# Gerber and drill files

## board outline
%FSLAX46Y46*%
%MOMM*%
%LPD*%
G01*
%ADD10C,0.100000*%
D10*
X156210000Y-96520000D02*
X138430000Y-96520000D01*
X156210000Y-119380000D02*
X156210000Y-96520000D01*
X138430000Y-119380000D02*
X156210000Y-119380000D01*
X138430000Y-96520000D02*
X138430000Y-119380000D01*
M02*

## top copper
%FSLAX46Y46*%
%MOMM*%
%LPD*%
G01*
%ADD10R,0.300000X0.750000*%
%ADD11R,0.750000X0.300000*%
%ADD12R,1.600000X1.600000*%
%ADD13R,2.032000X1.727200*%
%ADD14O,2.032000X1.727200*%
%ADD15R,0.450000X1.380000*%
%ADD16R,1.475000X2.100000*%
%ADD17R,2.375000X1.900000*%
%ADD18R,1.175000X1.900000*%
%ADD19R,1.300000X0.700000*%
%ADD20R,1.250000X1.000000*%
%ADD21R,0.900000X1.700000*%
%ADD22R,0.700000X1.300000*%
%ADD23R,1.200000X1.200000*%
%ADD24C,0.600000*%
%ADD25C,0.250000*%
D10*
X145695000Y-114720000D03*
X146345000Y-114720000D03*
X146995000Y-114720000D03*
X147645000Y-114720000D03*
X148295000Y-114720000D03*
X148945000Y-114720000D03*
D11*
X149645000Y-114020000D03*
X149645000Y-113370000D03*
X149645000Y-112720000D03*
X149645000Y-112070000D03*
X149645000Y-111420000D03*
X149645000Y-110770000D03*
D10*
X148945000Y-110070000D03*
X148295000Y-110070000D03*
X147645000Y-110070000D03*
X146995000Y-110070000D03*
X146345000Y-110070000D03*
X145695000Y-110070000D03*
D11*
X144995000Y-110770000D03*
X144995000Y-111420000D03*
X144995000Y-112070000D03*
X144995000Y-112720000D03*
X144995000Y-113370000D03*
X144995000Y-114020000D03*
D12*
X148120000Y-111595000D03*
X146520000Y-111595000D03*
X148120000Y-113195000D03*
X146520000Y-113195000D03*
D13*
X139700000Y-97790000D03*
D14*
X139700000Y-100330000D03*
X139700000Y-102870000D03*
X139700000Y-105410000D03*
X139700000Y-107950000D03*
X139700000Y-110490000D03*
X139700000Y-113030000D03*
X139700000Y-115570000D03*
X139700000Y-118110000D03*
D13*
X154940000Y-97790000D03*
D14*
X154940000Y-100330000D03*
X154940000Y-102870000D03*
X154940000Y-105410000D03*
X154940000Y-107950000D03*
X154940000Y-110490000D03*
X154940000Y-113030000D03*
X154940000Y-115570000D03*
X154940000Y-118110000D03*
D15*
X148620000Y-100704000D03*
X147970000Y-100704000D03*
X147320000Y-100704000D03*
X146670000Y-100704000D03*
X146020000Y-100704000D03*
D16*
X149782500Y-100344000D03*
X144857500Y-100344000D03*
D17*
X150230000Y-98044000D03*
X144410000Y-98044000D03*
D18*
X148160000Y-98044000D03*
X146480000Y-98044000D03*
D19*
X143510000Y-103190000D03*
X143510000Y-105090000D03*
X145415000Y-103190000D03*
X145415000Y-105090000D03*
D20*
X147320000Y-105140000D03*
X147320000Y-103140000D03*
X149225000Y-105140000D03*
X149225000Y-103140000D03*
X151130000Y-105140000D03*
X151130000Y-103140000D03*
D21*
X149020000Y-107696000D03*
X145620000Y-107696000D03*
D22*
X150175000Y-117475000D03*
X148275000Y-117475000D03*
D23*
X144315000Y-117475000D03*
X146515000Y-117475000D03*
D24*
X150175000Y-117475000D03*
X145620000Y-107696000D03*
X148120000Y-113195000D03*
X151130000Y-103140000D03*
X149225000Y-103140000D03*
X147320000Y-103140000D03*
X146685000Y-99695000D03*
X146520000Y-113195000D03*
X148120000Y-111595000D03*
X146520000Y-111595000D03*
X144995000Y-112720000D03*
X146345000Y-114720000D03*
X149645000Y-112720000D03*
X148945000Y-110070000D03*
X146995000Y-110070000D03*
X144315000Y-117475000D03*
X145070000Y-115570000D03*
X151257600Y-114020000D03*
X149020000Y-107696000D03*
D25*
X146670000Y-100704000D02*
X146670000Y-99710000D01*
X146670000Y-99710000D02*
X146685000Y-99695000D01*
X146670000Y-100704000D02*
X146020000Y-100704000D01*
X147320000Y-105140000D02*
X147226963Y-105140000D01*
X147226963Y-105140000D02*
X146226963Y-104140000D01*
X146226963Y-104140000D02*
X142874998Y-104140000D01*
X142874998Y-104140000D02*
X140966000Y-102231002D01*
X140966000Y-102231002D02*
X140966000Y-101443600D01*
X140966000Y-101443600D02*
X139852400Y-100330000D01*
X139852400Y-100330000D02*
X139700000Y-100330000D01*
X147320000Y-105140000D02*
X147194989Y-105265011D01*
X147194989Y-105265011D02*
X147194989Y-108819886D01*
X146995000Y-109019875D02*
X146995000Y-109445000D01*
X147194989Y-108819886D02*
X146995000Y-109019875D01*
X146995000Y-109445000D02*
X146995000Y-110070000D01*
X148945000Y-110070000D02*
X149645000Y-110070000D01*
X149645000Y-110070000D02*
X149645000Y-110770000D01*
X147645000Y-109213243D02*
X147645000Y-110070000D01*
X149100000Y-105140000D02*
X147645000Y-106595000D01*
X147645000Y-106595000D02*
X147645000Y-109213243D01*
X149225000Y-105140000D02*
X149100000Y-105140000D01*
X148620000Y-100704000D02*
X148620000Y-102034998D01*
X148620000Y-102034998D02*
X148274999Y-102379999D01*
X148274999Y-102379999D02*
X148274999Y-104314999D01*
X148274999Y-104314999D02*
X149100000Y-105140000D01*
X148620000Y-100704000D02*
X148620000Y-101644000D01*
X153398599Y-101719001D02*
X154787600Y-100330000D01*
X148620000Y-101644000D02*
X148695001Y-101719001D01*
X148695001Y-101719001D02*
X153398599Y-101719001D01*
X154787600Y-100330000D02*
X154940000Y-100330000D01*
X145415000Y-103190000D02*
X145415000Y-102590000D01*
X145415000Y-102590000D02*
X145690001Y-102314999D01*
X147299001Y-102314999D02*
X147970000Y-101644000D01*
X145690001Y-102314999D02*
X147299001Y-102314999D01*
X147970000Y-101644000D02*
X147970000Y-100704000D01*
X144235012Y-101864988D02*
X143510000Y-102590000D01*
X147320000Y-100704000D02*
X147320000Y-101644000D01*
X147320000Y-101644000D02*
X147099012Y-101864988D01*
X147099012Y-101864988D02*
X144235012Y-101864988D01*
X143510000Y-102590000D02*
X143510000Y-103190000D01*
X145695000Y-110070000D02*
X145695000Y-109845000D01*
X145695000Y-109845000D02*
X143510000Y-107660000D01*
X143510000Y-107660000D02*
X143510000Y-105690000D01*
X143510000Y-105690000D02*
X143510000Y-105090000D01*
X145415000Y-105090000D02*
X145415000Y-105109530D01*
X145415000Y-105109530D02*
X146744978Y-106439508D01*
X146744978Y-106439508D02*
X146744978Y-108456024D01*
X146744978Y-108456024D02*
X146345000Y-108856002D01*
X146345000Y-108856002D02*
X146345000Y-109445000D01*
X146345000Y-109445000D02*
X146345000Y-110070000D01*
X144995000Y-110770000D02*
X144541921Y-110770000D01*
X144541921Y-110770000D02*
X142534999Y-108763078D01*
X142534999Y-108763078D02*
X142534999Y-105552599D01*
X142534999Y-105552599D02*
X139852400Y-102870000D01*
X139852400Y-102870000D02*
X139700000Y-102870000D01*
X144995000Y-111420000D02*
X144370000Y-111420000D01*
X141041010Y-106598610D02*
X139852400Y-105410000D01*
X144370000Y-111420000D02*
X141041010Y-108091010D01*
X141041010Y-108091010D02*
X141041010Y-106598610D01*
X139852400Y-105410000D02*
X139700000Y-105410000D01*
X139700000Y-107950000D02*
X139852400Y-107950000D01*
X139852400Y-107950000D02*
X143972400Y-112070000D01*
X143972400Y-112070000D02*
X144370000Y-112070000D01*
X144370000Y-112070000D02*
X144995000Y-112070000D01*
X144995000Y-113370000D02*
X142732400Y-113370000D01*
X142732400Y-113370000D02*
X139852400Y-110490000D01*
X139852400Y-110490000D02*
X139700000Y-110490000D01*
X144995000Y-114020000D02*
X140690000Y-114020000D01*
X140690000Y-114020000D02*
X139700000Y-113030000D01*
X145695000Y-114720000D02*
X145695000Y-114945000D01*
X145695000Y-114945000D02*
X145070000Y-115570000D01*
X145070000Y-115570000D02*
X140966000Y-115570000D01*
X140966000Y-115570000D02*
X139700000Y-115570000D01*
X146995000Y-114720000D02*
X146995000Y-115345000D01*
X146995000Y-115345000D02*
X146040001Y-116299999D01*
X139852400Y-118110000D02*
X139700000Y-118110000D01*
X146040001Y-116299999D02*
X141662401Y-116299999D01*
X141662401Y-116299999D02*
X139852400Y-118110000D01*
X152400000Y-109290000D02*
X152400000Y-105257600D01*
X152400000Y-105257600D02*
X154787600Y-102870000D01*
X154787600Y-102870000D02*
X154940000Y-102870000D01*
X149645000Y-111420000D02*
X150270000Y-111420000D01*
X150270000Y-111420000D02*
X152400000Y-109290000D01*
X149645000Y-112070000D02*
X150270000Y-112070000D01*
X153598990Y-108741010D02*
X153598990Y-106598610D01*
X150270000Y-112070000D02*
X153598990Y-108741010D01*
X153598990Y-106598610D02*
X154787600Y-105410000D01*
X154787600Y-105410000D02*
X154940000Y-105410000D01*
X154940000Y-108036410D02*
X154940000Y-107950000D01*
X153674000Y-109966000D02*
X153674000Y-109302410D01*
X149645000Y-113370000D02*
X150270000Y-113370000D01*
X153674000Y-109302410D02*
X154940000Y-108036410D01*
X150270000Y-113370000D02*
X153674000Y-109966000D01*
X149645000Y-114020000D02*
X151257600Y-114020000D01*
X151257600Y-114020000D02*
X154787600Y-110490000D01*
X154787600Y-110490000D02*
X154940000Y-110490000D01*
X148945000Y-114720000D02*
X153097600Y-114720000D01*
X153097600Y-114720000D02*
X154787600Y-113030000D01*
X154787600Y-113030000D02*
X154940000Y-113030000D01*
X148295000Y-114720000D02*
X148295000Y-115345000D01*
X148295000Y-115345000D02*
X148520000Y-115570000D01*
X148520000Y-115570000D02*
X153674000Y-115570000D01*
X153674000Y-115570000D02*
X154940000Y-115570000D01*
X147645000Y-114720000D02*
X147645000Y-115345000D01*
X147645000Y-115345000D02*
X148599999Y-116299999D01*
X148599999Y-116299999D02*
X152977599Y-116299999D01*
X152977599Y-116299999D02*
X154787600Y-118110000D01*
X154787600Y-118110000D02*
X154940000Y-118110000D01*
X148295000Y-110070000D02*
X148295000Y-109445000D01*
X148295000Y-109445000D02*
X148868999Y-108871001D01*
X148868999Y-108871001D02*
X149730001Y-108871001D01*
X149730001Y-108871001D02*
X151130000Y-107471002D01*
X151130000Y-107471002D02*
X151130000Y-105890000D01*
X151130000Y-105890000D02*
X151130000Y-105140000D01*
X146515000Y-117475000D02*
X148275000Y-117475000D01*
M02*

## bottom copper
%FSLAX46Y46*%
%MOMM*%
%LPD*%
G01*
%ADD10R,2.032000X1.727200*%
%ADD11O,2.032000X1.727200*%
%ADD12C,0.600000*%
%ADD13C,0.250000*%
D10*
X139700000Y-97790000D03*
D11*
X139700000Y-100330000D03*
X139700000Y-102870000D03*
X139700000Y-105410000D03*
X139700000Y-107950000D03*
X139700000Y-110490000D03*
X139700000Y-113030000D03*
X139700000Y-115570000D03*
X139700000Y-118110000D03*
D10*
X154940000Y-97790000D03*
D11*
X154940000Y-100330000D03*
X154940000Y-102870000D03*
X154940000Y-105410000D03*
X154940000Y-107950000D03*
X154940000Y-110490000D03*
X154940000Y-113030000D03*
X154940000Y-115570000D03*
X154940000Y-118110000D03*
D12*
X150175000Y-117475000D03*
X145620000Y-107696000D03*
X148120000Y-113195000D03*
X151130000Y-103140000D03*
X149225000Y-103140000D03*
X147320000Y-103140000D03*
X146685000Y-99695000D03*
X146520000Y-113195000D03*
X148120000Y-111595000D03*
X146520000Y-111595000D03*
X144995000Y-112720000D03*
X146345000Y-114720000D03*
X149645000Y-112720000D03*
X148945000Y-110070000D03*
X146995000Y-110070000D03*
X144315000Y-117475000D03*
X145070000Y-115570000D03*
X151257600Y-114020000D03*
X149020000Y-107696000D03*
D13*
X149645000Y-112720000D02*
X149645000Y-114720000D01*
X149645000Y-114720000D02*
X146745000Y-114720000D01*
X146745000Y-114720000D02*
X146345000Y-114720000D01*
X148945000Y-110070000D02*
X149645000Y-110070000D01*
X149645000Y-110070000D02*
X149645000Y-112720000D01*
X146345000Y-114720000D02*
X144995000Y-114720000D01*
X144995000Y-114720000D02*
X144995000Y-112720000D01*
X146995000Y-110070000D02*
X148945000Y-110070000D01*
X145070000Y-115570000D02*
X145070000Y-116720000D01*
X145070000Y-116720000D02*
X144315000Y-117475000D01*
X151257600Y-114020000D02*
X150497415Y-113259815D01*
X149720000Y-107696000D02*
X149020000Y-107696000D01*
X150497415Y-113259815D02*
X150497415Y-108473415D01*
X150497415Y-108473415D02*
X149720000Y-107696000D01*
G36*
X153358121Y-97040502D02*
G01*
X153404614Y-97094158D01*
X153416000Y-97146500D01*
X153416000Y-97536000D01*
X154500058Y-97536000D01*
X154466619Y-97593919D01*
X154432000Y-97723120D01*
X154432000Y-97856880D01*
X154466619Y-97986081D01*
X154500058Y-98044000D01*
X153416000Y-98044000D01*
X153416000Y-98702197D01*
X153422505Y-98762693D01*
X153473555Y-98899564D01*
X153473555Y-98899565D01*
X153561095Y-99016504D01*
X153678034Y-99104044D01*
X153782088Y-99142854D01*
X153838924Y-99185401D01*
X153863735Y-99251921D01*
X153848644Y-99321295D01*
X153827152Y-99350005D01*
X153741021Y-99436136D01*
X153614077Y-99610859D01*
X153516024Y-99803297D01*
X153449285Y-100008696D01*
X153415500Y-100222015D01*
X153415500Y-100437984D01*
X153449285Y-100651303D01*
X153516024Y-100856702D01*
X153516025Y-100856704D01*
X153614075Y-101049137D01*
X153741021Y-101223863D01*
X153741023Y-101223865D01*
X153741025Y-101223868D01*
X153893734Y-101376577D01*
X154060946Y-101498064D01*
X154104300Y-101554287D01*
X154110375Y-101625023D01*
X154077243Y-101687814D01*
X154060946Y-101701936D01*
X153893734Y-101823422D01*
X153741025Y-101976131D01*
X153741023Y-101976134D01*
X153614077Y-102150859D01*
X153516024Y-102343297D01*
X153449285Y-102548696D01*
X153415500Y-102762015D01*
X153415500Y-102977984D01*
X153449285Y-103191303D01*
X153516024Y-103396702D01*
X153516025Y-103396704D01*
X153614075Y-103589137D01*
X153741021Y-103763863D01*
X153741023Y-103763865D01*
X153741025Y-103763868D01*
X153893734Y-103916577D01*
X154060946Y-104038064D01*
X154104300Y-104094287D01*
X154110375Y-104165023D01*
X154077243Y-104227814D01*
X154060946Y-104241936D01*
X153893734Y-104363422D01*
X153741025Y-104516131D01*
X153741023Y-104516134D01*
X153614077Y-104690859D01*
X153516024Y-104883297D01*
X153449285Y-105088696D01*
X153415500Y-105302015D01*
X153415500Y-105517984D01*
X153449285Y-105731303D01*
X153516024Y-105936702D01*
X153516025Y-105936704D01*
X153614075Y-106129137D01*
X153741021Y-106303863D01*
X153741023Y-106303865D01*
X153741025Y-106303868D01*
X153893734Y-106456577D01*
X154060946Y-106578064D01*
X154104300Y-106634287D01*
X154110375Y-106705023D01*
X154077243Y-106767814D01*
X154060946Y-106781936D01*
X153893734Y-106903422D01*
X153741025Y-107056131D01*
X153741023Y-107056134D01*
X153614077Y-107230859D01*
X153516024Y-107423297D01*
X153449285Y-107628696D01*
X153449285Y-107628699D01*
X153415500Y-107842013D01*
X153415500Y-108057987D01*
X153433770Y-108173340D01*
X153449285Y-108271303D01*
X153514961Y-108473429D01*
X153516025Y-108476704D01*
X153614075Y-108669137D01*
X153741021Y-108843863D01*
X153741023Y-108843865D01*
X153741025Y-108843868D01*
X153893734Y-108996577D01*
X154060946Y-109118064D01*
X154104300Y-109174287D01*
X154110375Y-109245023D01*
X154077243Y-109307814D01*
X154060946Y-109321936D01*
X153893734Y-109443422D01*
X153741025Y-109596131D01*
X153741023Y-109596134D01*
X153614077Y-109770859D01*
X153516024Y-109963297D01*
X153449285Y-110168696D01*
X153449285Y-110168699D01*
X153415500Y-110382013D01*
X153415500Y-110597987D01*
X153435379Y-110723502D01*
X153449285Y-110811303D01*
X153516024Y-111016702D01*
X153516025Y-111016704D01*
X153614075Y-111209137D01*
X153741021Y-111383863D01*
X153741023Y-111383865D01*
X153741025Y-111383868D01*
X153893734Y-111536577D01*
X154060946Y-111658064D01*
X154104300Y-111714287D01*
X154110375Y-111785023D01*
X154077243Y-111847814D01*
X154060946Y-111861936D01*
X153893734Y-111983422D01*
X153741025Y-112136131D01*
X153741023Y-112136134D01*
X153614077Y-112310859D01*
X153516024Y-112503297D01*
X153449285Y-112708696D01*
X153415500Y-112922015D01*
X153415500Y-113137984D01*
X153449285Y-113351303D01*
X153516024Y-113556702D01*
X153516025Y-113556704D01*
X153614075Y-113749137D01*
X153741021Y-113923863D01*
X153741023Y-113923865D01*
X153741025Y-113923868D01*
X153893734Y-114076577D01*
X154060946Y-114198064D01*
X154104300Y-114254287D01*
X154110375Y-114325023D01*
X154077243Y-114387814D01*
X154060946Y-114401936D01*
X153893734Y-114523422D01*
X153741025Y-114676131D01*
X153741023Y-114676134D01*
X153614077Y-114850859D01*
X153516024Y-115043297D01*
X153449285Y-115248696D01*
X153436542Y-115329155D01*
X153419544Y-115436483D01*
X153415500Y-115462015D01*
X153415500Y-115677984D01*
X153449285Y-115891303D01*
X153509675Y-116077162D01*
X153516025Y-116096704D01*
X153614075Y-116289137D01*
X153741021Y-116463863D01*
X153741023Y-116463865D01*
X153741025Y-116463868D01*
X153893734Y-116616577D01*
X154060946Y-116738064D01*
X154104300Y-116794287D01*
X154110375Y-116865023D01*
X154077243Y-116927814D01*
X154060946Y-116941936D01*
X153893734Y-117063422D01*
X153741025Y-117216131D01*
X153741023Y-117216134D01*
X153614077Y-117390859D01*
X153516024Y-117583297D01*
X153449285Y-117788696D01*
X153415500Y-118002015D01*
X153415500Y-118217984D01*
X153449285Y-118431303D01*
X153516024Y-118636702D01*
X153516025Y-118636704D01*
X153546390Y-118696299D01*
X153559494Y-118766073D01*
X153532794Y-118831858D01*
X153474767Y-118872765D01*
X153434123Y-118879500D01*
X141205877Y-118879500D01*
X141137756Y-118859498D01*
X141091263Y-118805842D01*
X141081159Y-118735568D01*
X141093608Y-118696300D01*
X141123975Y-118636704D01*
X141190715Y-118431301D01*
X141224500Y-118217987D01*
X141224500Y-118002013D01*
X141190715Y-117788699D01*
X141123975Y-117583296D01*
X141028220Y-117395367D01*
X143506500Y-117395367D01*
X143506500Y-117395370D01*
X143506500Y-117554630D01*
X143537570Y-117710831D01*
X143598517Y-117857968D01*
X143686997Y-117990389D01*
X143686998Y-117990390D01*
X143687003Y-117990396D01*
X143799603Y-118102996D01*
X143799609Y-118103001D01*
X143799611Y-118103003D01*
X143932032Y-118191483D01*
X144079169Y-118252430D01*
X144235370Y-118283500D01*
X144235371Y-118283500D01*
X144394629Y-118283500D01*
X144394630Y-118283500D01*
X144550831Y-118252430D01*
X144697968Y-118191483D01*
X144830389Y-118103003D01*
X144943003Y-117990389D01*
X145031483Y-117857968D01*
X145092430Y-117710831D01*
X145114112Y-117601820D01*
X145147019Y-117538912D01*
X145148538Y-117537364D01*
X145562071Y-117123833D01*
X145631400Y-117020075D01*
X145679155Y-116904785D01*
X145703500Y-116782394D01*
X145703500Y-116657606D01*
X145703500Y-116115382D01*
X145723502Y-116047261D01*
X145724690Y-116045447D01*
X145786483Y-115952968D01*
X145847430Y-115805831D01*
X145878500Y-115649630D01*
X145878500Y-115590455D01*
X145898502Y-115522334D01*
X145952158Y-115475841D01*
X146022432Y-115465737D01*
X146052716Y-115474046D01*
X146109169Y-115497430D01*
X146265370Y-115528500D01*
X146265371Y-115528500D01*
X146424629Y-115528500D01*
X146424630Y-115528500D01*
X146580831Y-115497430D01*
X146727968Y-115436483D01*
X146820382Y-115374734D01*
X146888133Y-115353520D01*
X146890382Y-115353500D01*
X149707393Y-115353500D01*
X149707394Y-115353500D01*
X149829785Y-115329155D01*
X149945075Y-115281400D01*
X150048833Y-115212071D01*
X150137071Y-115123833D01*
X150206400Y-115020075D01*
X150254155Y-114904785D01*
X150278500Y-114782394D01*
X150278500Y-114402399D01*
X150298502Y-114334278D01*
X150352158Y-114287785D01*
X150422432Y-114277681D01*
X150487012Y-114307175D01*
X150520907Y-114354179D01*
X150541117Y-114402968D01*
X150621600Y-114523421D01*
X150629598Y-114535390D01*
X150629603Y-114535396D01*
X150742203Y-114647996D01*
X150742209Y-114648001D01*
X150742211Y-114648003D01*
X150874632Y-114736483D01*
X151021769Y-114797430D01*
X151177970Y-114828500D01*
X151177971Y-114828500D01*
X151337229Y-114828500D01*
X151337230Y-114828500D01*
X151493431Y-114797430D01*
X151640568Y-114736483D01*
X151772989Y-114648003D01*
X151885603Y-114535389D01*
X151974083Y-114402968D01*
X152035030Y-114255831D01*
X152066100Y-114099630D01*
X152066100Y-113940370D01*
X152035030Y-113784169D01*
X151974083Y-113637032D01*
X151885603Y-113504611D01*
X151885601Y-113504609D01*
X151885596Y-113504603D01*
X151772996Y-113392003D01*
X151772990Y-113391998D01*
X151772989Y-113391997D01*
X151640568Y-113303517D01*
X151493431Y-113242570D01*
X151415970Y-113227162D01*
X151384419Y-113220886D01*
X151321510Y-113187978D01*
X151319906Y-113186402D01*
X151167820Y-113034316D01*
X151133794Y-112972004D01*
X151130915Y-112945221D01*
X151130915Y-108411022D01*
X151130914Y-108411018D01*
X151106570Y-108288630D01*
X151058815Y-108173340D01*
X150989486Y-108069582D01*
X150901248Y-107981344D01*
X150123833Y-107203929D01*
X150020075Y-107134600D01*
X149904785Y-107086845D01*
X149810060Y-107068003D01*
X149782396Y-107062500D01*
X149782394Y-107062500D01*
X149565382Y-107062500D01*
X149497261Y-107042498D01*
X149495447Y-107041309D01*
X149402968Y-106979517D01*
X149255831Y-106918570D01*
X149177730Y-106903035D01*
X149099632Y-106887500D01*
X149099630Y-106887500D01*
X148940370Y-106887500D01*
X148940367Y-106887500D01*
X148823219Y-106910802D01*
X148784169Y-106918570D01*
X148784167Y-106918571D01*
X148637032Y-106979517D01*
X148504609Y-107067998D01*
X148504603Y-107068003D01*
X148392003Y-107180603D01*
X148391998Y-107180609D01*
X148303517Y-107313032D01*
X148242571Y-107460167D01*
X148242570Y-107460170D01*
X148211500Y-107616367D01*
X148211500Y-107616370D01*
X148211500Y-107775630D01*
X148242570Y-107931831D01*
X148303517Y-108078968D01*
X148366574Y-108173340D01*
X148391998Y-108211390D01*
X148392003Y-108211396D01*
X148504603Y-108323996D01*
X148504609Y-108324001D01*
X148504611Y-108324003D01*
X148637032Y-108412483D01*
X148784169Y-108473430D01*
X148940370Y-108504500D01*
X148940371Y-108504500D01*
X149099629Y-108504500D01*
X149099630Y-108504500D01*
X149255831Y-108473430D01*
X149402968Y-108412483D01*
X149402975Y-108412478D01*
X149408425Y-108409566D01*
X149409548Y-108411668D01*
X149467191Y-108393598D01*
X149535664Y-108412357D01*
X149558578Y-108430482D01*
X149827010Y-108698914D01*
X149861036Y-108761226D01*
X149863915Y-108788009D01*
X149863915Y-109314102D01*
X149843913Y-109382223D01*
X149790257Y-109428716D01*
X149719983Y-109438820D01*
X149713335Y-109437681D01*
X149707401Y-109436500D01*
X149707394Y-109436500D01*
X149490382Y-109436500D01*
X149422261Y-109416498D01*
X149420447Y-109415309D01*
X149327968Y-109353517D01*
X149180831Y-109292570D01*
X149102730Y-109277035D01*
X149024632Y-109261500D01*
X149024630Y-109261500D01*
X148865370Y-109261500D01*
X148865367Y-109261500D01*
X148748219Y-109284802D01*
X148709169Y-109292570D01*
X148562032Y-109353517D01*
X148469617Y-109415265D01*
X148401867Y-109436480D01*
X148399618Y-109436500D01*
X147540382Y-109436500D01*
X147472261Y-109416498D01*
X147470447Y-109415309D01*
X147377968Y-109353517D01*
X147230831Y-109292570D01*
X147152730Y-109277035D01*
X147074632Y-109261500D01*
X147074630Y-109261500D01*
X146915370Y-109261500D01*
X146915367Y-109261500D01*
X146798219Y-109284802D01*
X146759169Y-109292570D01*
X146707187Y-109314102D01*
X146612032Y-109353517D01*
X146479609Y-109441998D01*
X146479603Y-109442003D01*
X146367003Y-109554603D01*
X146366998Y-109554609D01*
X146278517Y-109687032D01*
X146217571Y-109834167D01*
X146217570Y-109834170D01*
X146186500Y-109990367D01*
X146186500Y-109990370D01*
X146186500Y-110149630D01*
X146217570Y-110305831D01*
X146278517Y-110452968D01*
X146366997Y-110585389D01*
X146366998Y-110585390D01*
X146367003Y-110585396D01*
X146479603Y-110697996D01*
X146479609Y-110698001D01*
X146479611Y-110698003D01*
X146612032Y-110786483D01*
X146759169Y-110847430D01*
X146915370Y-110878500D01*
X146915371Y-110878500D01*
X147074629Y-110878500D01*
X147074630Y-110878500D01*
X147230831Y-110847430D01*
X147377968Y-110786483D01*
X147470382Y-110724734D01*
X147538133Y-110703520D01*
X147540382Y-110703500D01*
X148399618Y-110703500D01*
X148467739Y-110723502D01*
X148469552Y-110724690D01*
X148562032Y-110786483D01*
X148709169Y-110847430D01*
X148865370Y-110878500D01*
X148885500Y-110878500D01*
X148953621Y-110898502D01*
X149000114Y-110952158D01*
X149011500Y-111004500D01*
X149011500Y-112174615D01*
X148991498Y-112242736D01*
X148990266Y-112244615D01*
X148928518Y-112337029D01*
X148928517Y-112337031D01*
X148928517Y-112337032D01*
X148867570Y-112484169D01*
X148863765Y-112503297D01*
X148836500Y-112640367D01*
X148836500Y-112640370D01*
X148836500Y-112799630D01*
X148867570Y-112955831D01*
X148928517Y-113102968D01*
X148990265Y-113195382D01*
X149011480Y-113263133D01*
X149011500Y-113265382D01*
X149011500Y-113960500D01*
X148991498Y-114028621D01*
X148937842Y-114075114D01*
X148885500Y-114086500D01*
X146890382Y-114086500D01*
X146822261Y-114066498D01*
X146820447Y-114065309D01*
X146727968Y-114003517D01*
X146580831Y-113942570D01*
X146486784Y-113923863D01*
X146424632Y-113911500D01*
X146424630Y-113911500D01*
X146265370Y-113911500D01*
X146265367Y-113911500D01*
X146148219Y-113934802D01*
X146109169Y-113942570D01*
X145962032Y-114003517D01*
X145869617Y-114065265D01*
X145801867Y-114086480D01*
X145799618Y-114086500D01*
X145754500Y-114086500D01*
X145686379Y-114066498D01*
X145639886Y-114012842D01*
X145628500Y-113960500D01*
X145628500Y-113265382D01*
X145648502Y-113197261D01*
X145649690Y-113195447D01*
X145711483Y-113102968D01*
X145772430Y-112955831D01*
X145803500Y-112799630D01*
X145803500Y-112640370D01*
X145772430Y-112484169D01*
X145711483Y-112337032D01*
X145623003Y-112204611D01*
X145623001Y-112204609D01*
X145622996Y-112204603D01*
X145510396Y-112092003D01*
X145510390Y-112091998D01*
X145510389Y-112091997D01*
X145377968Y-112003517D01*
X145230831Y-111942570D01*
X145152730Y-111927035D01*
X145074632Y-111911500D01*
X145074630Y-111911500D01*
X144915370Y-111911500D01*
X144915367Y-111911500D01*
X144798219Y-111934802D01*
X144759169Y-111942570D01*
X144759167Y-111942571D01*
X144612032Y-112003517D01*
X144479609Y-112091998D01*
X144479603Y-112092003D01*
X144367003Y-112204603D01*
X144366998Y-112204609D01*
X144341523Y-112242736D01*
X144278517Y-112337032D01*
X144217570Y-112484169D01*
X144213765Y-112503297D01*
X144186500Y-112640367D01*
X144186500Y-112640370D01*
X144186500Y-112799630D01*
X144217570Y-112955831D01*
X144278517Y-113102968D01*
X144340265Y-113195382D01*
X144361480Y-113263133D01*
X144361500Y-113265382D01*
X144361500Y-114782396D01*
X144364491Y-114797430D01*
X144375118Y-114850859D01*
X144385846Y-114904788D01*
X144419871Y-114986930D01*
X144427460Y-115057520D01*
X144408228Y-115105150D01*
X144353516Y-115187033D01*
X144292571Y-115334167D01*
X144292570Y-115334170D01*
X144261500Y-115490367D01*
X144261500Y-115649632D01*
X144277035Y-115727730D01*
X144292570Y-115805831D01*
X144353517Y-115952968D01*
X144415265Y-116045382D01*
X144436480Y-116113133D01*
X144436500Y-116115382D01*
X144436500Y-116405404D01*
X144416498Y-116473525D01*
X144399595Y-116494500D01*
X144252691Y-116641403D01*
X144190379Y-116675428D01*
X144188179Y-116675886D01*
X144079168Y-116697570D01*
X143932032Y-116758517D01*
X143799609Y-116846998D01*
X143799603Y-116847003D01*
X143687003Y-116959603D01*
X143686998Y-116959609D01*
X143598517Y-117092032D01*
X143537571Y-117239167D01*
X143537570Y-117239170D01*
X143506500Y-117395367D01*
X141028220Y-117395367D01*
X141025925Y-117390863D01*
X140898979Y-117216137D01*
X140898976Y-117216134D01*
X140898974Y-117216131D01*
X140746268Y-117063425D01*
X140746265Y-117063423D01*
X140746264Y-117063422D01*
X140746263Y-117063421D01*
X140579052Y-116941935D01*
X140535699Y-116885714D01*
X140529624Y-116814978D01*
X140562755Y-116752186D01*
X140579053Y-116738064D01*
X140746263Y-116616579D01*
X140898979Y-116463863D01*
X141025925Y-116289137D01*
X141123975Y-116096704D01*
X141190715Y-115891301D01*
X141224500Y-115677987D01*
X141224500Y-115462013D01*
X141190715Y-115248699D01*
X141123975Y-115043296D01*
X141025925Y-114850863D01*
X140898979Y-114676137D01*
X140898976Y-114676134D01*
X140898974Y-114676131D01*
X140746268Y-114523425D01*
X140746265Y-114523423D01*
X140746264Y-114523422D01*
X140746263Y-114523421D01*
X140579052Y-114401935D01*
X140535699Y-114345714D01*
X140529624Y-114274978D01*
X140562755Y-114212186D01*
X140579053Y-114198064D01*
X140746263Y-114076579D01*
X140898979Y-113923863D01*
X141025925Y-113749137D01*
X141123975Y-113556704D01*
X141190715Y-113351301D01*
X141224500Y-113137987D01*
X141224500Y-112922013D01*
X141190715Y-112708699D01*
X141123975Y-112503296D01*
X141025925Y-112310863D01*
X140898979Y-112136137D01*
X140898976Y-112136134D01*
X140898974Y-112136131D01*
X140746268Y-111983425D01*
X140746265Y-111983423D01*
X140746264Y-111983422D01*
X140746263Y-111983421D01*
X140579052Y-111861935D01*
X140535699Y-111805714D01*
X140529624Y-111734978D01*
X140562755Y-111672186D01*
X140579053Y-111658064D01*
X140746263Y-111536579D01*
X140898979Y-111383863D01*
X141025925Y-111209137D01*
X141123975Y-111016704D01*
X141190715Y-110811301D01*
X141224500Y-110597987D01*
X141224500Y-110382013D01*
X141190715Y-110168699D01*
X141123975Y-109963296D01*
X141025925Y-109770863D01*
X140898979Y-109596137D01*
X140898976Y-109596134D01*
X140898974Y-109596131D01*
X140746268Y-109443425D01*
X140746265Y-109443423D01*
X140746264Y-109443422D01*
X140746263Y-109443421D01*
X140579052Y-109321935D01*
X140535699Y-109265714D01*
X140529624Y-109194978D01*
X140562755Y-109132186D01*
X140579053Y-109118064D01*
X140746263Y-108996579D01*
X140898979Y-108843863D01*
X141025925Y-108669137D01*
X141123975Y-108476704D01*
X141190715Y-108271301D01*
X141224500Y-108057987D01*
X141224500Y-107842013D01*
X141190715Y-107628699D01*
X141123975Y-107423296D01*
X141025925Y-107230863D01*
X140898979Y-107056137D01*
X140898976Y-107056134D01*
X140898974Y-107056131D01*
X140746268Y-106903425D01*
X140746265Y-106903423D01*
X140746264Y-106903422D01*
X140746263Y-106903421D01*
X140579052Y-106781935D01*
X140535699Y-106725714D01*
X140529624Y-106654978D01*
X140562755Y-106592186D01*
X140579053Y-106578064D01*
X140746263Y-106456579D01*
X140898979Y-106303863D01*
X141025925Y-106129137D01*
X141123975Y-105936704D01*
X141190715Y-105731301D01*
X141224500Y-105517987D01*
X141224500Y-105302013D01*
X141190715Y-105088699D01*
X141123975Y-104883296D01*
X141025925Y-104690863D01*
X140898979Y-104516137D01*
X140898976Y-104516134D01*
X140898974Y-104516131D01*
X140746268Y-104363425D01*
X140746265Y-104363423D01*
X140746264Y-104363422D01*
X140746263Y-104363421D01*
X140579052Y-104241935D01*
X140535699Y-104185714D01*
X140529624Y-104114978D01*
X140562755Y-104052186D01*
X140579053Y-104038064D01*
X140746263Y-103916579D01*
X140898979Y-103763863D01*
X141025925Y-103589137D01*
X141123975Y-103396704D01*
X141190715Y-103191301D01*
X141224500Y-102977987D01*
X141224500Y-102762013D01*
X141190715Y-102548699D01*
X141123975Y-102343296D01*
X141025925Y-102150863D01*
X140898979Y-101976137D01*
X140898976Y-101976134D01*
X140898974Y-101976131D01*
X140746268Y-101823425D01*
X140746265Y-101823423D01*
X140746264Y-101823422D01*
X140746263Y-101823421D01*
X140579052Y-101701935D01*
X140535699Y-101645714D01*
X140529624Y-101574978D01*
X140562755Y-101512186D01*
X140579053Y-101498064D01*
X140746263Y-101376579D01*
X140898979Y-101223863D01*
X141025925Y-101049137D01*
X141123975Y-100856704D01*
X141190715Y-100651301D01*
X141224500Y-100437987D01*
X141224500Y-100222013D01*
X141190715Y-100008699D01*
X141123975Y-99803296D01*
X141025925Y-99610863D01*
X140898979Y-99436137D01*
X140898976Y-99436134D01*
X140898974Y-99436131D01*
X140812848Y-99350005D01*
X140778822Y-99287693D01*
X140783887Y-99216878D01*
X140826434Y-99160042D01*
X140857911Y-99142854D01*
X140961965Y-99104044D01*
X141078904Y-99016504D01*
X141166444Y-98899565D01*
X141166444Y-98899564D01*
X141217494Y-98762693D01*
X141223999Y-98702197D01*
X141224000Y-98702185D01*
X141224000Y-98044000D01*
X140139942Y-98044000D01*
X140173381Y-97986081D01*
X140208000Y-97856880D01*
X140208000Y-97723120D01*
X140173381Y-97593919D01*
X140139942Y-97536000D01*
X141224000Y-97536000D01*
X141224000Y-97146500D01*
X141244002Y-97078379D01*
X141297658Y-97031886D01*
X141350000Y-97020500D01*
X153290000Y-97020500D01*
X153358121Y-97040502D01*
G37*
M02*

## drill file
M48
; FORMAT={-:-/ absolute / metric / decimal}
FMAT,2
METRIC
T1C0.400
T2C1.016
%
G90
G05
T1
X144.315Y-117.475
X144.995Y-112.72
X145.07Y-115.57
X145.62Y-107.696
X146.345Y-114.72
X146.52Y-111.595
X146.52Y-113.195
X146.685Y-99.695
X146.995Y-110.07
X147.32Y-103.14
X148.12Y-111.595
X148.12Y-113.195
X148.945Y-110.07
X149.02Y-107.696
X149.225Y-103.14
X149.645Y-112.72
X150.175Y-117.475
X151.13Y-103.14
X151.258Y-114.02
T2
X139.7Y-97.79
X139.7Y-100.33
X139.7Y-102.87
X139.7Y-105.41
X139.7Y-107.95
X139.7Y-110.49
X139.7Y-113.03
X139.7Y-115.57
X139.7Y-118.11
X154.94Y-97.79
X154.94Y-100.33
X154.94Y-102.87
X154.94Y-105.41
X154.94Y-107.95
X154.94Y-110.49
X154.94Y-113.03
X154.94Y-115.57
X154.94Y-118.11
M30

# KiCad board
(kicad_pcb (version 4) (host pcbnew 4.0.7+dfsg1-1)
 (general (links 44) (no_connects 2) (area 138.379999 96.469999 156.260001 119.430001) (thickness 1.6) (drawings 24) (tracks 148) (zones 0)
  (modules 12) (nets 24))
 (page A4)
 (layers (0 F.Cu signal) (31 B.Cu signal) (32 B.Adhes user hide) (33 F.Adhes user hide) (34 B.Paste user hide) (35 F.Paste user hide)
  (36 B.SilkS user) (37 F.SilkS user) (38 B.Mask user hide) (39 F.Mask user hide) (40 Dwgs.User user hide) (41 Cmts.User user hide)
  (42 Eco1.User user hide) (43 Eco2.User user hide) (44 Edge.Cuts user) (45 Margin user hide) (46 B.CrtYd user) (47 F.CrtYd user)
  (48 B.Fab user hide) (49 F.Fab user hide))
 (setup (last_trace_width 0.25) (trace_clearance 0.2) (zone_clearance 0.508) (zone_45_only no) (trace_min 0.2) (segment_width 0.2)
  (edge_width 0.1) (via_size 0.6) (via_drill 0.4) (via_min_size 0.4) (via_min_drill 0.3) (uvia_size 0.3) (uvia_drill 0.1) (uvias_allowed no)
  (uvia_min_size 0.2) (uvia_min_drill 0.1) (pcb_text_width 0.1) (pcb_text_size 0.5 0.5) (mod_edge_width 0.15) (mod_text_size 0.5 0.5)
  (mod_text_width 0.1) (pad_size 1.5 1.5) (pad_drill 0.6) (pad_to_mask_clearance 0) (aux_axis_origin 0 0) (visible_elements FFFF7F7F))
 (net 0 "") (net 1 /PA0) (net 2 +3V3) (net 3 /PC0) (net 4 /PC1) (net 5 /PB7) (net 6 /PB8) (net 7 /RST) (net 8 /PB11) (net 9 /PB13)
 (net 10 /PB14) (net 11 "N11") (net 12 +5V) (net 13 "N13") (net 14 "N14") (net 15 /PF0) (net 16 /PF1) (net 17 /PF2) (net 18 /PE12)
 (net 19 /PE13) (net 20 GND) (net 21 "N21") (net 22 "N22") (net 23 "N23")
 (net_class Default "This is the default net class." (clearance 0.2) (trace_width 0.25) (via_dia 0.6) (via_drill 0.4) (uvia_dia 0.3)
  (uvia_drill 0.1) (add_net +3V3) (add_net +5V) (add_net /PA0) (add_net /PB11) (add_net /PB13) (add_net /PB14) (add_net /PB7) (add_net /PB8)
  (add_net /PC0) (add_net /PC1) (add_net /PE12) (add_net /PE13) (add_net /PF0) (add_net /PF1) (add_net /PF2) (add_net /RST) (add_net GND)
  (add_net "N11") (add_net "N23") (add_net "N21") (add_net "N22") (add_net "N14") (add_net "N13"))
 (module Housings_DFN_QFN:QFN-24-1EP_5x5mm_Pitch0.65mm (layer F.Cu) (at 147.32 112.395 90)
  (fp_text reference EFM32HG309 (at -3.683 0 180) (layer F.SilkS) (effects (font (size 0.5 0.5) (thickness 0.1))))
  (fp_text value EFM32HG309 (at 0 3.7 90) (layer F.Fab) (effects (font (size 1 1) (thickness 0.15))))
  (pad 1 smd rect (at -2.325 -1.625 90) (size 0.75 0.3) (layers F.Cu F.Paste F.Mask) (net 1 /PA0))
  (pad 2 smd rect (at -2.325 -0.975 90) (size 0.75 0.3) (layers F.Cu F.Paste F.Mask) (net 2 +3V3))
  (pad 3 smd rect (at -2.325 -0.325 90) (size 0.75 0.3) (layers F.Cu F.Paste F.Mask) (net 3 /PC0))
  (pad 4 smd rect (at -2.325 0.325 90) (size 0.75 0.3) (layers F.Cu F.Paste F.Mask) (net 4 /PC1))
  (pad 5 smd rect (at -2.325 0.975 90) (size 0.75 0.3) (layers F.Cu F.Paste F.Mask) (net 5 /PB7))
  (pad 6 smd rect (at -2.325 1.625 90) (size 0.75 0.3) (layers F.Cu F.Paste F.Mask) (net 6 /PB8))
  (pad 7 smd rect (at -1.625 2.325 180) (size 0.75 0.3) (layers F.Cu F.Paste F.Mask) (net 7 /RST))
  (pad 8 smd rect (at -0.975 2.325 180) (size 0.75 0.3) (layers F.Cu F.Paste F.Mask) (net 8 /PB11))
  (pad 9 smd rect (at -0.325 2.325 180) (size 0.75 0.3) (layers F.Cu F.Paste F.Mask) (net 2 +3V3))
  (pad 10 smd rect (at 0.325 2.325 180) (size 0.75 0.3) (layers F.Cu F.Paste F.Mask) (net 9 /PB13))
  (pad 11 smd rect (at 0.975 2.325 180) (size 0.75 0.3) (layers F.Cu F.Paste F.Mask) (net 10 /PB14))
  (pad 12 smd rect (at 1.625 2.325 180) (size 0.75 0.3) (layers F.Cu F.Paste F.Mask) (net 2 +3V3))
  (pad 13 smd rect (at 2.325 1.625 90) (size 0.75 0.3) (layers F.Cu F.Paste F.Mask) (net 2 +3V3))
  (pad 14 smd rect (at 2.325 0.975 90) (size 0.75 0.3) (layers F.Cu F.Paste F.Mask) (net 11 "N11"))
  (pad 15 smd rect (at 2.325 0.325 90) (size 0.75 0.3) (layers F.Cu F.Paste F.Mask) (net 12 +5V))
  (pad 16 smd rect (at 2.325 -0.325 90) (size 0.75 0.3) (layers F.Cu F.Paste F.Mask) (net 2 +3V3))
  (pad 17 smd rect (at 2.325 -0.975 90) (size 0.75 0.3) (layers F.Cu F.Paste F.Mask) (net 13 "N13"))
  (pad 18 smd rect (at 2.325 -1.625 90) (size 0.75 0.3) (layers F.Cu F.Paste F.Mask) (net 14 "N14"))
  (pad 19 smd rect (at 1.625 -2.325 180) (size 0.75 0.3) (layers F.Cu F.Paste F.Mask) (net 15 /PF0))
  (pad 20 smd rect (at 0.975 -2.325 180) (size 0.75 0.3) (layers F.Cu F.Paste F.Mask) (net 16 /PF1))
  (pad 21 smd rect (at 0.325 -2.325 180) (size 0.75 0.3) (layers F.Cu F.Paste F.Mask) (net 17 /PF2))
  (pad 22 smd rect (at -0.325 -2.325 180) (size 0.75 0.3) (layers F.Cu F.Paste F.Mask) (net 2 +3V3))
  (pad 23 smd rect (at -0.975 -2.325 180) (size 0.75 0.3) (layers F.Cu F.Paste F.Mask) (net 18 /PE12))
  (pad 24 smd rect (at -1.625 -2.325 180) (size 0.75 0.3) (layers F.Cu F.Paste F.Mask) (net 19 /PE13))
  (pad 25 smd rect (at 0.8 0.8 90) (size 1.6 1.6) (layers F.Cu F.Paste F.Mask) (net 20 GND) (solder_paste_margin_ratio -0.2))
  (pad 25 smd rect (at 0.8 -0.8 90) (size 1.6 1.6) (layers F.Cu F.Paste F.Mask) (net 20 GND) (solder_paste_margin_ratio -0.2))
  (pad 25 smd rect (at -0.8 0.8 90) (size 1.6 1.6) (layers F.Cu F.Paste F.Mask) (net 20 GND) (solder_paste_margin_ratio -0.2))
  (pad 25 smd rect (at -0.8 -0.8 90) (size 1.6 1.6) (layers F.Cu F.Paste F.Mask) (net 20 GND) (solder_paste_margin_ratio -0.2)))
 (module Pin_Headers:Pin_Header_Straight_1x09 (layer B.Cu) (at 139.7 97.79 180)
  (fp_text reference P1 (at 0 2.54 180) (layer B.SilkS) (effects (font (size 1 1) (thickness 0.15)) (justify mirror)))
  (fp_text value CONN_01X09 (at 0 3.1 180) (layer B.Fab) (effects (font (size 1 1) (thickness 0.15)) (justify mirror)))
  (pad 1 thru_hole rect (at 0 0 180) (size 2.032 1.7272) (drill 1.016) (layers *.Cu *.Mask) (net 20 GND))
  (pad 2 thru_hole oval (at 0 -2.54 180) (size 2.032 1.7272) (drill 1.016) (layers *.Cu *.Mask) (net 2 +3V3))
  (pad 3 thru_hole oval (at 0 -5.08 180) (size 2.032 1.7272) (drill 1.016) (layers *.Cu *.Mask) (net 15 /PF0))
  (pad 4 thru_hole oval (at 0 -7.62 180) (size 2.032 1.7272) (drill 1.016) (layers *.Cu *.Mask) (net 16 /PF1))
  (pad 5 thru_hole oval (at 0 -10.16 180) (size 2.032 1.7272) (drill 1.016) (layers *.Cu *.Mask) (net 17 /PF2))
  (pad 6 thru_hole oval (at 0 -12.7 180) (size 2.032 1.7272) (drill 1.016) (layers *.Cu *.Mask) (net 18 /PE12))
  (pad 7 thru_hole oval (at 0 -15.24 180) (size 2.032 1.7272) (drill 1.016) (layers *.Cu *.Mask) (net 19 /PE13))
  (pad 8 thru_hole oval (at 0 -17.78 180) (size 2.032 1.7272) (drill 1.016) (layers *.Cu *.Mask) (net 1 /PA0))
  (pad 9 thru_hole oval (at 0 -20.32 180) (size 2.032 1.7272) (drill 1.016) (layers *.Cu *.Mask) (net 3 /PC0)))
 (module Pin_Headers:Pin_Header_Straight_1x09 (layer B.Cu) (at 154.94 97.79 180)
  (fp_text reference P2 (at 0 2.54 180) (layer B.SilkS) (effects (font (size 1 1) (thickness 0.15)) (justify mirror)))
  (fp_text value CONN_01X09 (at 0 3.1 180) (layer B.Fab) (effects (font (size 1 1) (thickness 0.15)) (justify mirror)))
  (pad 1 thru_hole rect (at 0 0 180) (size 2.032 1.7272) (drill 1.016) (layers *.Cu *.Mask) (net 20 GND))
  (pad 2 thru_hole oval (at 0 -2.54 180) (size 2.032 1.7272) (drill 1.016) (layers *.Cu *.Mask) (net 12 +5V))
  (pad 3 thru_hole oval (at 0 -5.08 180) (size 2.032 1.7272) (drill 1.016) (layers *.Cu *.Mask) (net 10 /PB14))
  (pad 4 thru_hole oval (at 0 -7.62 180) (size 2.032 1.7272) (drill 1.016) (layers *.Cu *.Mask) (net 9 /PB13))
  (pad 5 thru_hole oval (at 0 -10.16 180) (size 2.032 1.7272) (drill 1.016) (layers *.Cu *.Mask) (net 8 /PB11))
  (pad 6 thru_hole oval (at 0 -12.7 180) (size 2.032 1.7272) (drill 1.016) (layers *.Cu *.Mask) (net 7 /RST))
  (pad 7 thru_hole oval (at 0 -15.24 180) (size 2.032 1.7272) (drill 1.016) (layers *.Cu *.Mask) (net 6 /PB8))
  (pad 8 thru_hole oval (at 0 -17.78 180) (size 2.032 1.7272) (drill 1.016) (layers *.Cu *.Mask) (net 5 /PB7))
  (pad 9 thru_hole oval (at 0 -20.32 180) (size 2.032 1.7272) (drill 1.016) (layers *.Cu *.Mask) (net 4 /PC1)))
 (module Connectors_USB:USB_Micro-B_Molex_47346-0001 (layer F.Cu) (at 147.32 98.044 180)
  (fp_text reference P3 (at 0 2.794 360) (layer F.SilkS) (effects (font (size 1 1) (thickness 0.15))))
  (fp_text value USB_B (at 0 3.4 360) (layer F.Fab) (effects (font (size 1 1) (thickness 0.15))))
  (pad 1 smd rect (at -1.3 -2.66 180) (size 0.45 1.38) (layers F.Cu F.Paste F.Mask) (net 12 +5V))
  (pad 2 smd rect (at -0.65 -2.66 180) (size 0.45 1.38) (layers F.Cu F.Paste F.Mask) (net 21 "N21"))
  (pad 3 smd rect (at 0 -2.66 180) (size 0.45 1.38) (layers F.Cu F.Paste F.Mask) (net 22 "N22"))
  (pad 4 smd rect (at 0.65 -2.66 180) (size 0.45 1.38) (layers F.Cu F.Paste F.Mask) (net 20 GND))
  (pad 5 smd rect (at 1.3 -2.66 180) (size 0.45 1.38) (layers F.Cu F.Paste F.Mask) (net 20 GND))
  (pad 6 smd rect (at -2.4625 -2.3 180) (size 1.475 2.1) (layers F.Cu F.Paste F.Mask))
  (pad 6 smd rect (at 2.4625 -2.3 180) (size 1.475 2.1) (layers F.Cu F.Paste F.Mask))
  (pad 6 smd rect (at -2.91 0 180) (size 2.375 1.9) (layers F.Cu F.Paste F.Mask))
  (pad 6 smd rect (at 2.91 0 180) (size 2.375 1.9) (layers F.Cu F.Paste F.Mask))
  (pad 6 smd rect (at -0.84 0 180) (size 1.175 1.9) (layers F.Cu F.Paste F.Mask))
  (pad 6 smd rect (at 0.84 0 180) (size 1.175 1.9) (layers F.Cu F.Paste F.Mask)))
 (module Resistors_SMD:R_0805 (layer F.Cu) (at 143.51 104.14 270)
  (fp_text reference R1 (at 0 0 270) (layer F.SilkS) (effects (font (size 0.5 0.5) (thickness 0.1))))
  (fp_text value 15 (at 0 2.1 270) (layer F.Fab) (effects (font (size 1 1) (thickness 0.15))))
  (pad 1 smd rect (at -0.95 0 270) (size 0.7 1.3) (layers F.Cu F.Paste F.Mask) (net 22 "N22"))
  (pad 2 smd rect (at 0.95 0 270) (size 0.7 1.3) (layers F.Cu F.Paste F.Mask) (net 14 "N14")))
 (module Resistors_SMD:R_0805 (layer F.Cu) (at 145.415 104.14 270)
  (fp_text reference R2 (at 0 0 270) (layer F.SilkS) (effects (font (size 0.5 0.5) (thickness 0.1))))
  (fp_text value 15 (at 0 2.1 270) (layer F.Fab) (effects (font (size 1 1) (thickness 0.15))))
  (pad 1 smd rect (at -0.95 0 270) (size 0.7 1.3) (layers F.Cu F.Paste F.Mask) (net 21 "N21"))
  (pad 2 smd rect (at 0.95 0 270) (size 0.7 1.3) (layers F.Cu F.Paste F.Mask) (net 13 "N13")))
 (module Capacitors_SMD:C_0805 (layer F.Cu) (at 147.32 104.14 90)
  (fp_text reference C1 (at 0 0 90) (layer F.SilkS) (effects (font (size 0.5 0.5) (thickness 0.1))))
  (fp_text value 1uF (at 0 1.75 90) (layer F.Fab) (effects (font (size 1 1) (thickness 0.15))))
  (pad 1 smd rect (at -1 0 90) (size 1 1.25) (layers F.Cu F.Paste F.Mask) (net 2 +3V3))
  (pad 2 smd rect (at 1 0 90) (size 1 1.25) (layers F.Cu F.Paste F.Mask) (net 20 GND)))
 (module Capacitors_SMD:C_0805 (layer F.Cu) (at 149.225 104.14 90)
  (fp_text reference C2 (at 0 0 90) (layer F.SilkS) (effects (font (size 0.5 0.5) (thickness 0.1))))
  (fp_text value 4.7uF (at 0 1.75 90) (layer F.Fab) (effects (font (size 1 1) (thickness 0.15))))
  (pad 1 smd rect (at -1 0 90) (size 1 1.25) (layers F.Cu F.Paste F.Mask) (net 12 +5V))
  (pad 2 smd rect (at 1 0 90) (size 1 1.25) (layers F.Cu F.Paste F.Mask) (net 20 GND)))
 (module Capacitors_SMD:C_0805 (layer F.Cu) (at 151.13 104.14 90)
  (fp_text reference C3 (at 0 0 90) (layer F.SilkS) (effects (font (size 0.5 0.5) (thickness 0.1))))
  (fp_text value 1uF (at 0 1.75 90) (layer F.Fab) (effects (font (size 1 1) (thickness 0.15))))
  (pad 1 smd rect (at -1 0 90) (size 1 1.25) (layers F.Cu F.Paste F.Mask) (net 11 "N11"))
  (pad 2 smd rect (at 1 0 90) (size 1 1.25) (layers F.Cu F.Paste F.Mask) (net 20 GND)))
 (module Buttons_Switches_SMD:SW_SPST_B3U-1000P (layer F.Cu) (at 147.32 107.696 180)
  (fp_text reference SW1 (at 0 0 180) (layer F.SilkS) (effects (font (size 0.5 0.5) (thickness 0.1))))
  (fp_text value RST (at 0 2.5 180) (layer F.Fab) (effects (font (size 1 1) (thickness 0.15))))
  (pad 1 smd rect (at -1.7 0 180) (size 0.9 1.7) (layers F.Cu F.Paste F.Mask) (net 7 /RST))
  (pad 2 smd rect (at 1.7 0 180) (size 0.9 1.7) (layers F.Cu F.Paste F.Mask) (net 20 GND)))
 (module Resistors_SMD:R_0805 (layer F.Cu) (at 149.225 117.475 180)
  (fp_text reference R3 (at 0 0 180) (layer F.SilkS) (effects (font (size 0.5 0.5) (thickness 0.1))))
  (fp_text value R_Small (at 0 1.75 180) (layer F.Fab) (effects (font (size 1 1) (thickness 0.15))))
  (pad 1 smd rect (at -0.95 0 180) (size 0.7 1.3) (layers F.Cu F.Paste F.Mask) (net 20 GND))
  (pad 2 smd rect (at 0.95 0 180) (size 0.7 1.3) (layers F.Cu F.Paste F.Mask) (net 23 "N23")))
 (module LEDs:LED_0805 (layer F.Cu) (at 145.415 117.475 180)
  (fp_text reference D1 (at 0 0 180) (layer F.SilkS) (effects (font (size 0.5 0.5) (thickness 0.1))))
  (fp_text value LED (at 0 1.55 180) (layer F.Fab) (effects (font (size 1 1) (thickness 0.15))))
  (pad 2 smd rect (at 1.1 0) (size 1.2 1.2) (layers F.Cu F.Paste F.Mask) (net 1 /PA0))
  (pad 1 smd rect (at -1.1 0) (size 1.2 1.2) (layers F.Cu F.Paste F.Mask) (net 23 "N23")))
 (gr_line (start 156.21 96.52) (end 138.43 96.52) (layer Edge.Cuts) (width 0.1))
 (gr_line (start 156.21 119.38) (end 156.21 96.52) (layer Edge.Cuts) (width 0.1))
 (gr_line (start 138.43 119.38) (end 156.21 119.38) (layer Edge.Cuts) (width 0.1))
 (gr_line (start 138.43 96.52) (end 138.43 119.38) (layer Edge.Cuts) (width 0.1))
 (via (at 150.175 117.475) (size 0.6) (drill 0.4) (layers F.Cu B.Cu) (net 20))
 (via (at 145.62 107.696) (size 0.6) (drill 0.4) (layers F.Cu B.Cu) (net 20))
 (via (at 148.12 113.195) (size 0.6) (drill 0.4) (layers F.Cu B.Cu) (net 20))
 (via (at 151.13 103.14) (size 0.6) (drill 0.4) (layers F.Cu B.Cu) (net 20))
 (via (at 149.225 103.14) (size 0.6) (drill 0.4) (layers F.Cu B.Cu) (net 20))
 (via (at 147.32 103.14) (size 0.6) (drill 0.4) (layers F.Cu B.Cu) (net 20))
 (segment (start 146.67 100.704) (end 146.67 99.71) (width 0.25) (layer F.Cu) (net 20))
 (segment (start 146.67 99.71) (end 146.685 99.695) (width 0.25) (layer F.Cu) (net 20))
 (via (at 146.685 99.695) (size 0.6) (drill 0.4) (layers F.Cu B.Cu) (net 20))
 (via (at 146.52 113.195) (size 0.6) (drill 0.4) (layers F.Cu B.Cu) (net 20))
 (via (at 148.12 111.595) (size 0.6) (drill 0.4) (layers F.Cu B.Cu) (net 20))
 (via (at 146.52 111.595) (size 0.6) (drill 0.4) (layers F.Cu B.Cu) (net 20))
 (segment (start 146.67 100.704) (end 146.02 100.704) (width 0.25) (layer F.Cu) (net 20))
 (segment (start 147.32 105.14) (end 147.226963 105.14) (width 0.25) (layer F.Cu) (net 2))
 (segment (start 147.226963 105.14) (end 146.226963 104.14) (width 0.25) (layer F.Cu) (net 2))
 (segment (start 146.226963 104.14) (end 142.874998 104.14) (width 0.25) (layer F.Cu) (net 2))
 (segment (start 142.874998 104.14) (end 140.966 102.231002) (width 0.25) (layer F.Cu) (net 2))
 (segment (start 140.966 102.231002) (end 140.966 101.4436) (width 0.25) (layer F.Cu) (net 2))
 (segment (start 140.966 101.4436) (end 139.8524 100.33) (width 0.25) (layer F.Cu) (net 2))
 (segment (start 139.8524 100.33) (end 139.7 100.33) (width 0.25) (layer F.Cu) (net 2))
 (segment (start 147.32 105.14) (end 147.194989 105.265011) (width 0.25) (layer F.Cu) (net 2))
 (segment (start 147.194989 105.265011) (end 147.194989 108.819886) (width 0.25) (layer F.Cu) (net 2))
 (segment (start 146.995 109.019875) (end 146.995 109.445) (width 0.25) (layer F.Cu) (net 2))
 (segment (start 147.194989 108.819886) (end 146.995 109.019875) (width 0.25) (layer F.Cu) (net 2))
 (segment (start 146.995 109.445) (end 146.995 110.07) (width 0.25) (layer F.Cu) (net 2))
 (segment (start 149.645 112.72) (end 149.645 114.72) (width 0.25) (layer B.Cu) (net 2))
 (segment (start 149.645 114.72) (end 146.745 114.72) (width 0.25) (layer B.Cu) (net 2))
 (segment (start 146.745 114.72) (end 146.345 114.72) (width 0.25) (layer B.Cu) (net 2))
 (segment (start 148.945 110.07) (end 149.645 110.07) (width 0.25) (layer F.Cu) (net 2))
 (segment (start 149.645 110.07) (end 149.645 110.77) (width 0.25) (layer F.Cu) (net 2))
 (segment (start 148.945 110.07) (end 149.645 110.07) (width 0.25) (layer B.Cu) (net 2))
 (segment (start 149.645 110.07) (end 149.645 112.72) (width 0.25) (layer B.Cu) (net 2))
 (segment (start 146.345 114.72) (end 144.995 114.72) (width 0.25) (layer B.Cu) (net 2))
 (segment (start 144.995 114.72) (end 144.995 112.72) (width 0.25) (layer B.Cu) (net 2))
 (via (at 144.995 112.72) (size 0.6) (drill 0.4) (layers F.Cu B.Cu) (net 2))
 (via (at 146.345 114.72) (size 0.6) (drill 0.4) (layers F.Cu B.Cu) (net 2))
 (via (at 149.645 112.72) (size 0.6) (drill 0.4) (layers F.Cu B.Cu) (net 2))
 (segment (start 146.995 110.07) (end 148.945 110.07) (width 0.25) (layer B.Cu) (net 2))
 (via (at 148.945 110.07) (size 0.6) (drill 0.4) (layers F.Cu B.Cu) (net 2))
 (via (at 146.995 110.07) (size 0.6) (drill 0.4) (layers F.Cu B.Cu) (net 2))
 (segment (start 147.645 109.213243) (end 147.645 110.07) (width 0.25) (layer F.Cu) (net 12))
 (segment (start 149.1 105.14) (end 147.645 106.595) (width 0.25) (layer F.Cu) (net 12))
 (segment (start 147.645 106.595) (end 147.645 109.213243) (width 0.25) (layer F.Cu) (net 12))
 (segment (start 149.225 105.14) (end 149.1 105.14) (width 0.25) (layer F.Cu) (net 12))
 (segment (start 148.62 100.704) (end 148.62 102.034998) (width 0.25) (layer F.Cu) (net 12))
 (segment (start 148.62 102.034998) (end 148.274999 102.379999) (width 0.25) (layer F.Cu) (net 12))
 (segment (start 148.274999 102.379999) (end 148.274999 104.314999) (width 0.25) (layer F.Cu) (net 12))
 (segment (start 148.274999 104.314999) (end 149.1 105.14) (width 0.25) (layer F.Cu) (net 12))
 (segment (start 148.62 100.704) (end 148.62 101.644) (width 0.25) (layer F.Cu) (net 12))
 (segment (start 153.398599 101.719001) (end 154.7876 100.33) (width 0.25) (layer F.Cu) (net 12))
 (segment (start 148.62 101.644) (end 148.695001 101.719001) (width 0.25) (layer F.Cu) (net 12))
 (segment (start 148.695001 101.719001) (end 153.398599 101.719001) (width 0.25) (layer F.Cu) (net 12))
 (segment (start 154.7876 100.33) (end 154.94 100.33) (width 0.25) (layer F.Cu) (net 12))
 (segment (start 145.415 103.19) (end 145.415 102.59) (width 0.25) (layer F.Cu) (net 21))
 (segment (start 145.415 102.59) (end 145.690001 102.314999) (width 0.25) (layer F.Cu) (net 21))
 (segment (start 147.299001 102.314999) (end 147.97 101.644) (width 0.25) (layer F.Cu) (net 21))
 (segment (start 145.690001 102.314999) (end 147.299001 102.314999) (width 0.25) (layer F.Cu) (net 21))
 (segment (start 147.97 101.644) (end 147.97 100.704) (width 0.25) (layer F.Cu) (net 21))
 (segment (start 144.235012 101.864988) (end 143.51 102.59) (width 0.25) (layer F.Cu) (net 22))
 (segment (start 147.32 100.704) (end 147.32 101.644) (width 0.25) (layer F.Cu) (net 22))
 (segment (start 147.32 101.644) (end 147.099012 101.864988) (width 0.25) (layer F.Cu) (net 22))
 (segment (start 147.099012 101.864988) (end 144.235012 101.864988) (width 0.25) (layer F.Cu) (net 22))
 (segment (start 143.51 102.59) (end 143.51 103.19) (width 0.25) (layer F.Cu) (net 22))
 (segment (start 145.695 110.07) (end 145.695 109.845) (width 0.25) (layer F.Cu) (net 14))
 (segment (start 145.695 109.845) (end 143.51 107.66) (width 0.25) (layer F.Cu) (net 14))
 (segment (start 143.51 107.66) (end 143.51 105.69) (width 0.25) (layer F.Cu) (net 14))
 (segment (start 143.51 105.69) (end 143.51 105.09) (width 0.25) (layer F.Cu) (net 14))
 (segment (start 145.415 105.09) (end 145.415 105.10953) (width 0.25) (layer F.Cu) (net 13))
 (segment (start 145.415 105.10953) (end 146.744978 106.439508) (width 0.25) (layer F.Cu) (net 13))
 (segment (start 146.744978 106.439508) (end 146.744978 108.456024) (width 0.25) (layer F.Cu) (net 13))
 (segment (start 146.744978 108.456024) (end 146.345 108.856002) (width 0.25) (layer F.Cu) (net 13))
 (segment (start 146.345 108.856002) (end 146.345 109.445) (width 0.25) (layer F.Cu) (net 13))
 (segment (start 146.345 109.445) (end 146.345 110.07) (width 0.25) (layer F.Cu) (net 13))
 (segment (start 144.995 110.77) (end 144.541921 110.77) (width 0.25) (layer F.Cu) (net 15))
 (segment (start 144.541921 110.77) (end 142.534999 108.763078) (width 0.25) (layer F.Cu) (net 15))
 (segment (start 142.534999 108.763078) (end 142.534999 105.552599) (width 0.25) (layer F.Cu) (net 15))
 (segment (start 142.534999 105.552599) (end 139.8524 102.87) (width 0.25) (layer F.Cu) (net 15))
 (segment (start 139.8524 102.87) (end 139.7 102.87) (width 0.25) (layer F.Cu) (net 15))
 (segment (start 144.995 111.42) (end 144.37 111.42) (width 0.25) (layer F.Cu) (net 16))
 (segment (start 141.04101 106.59861) (end 139.8524 105.41) (width 0.25) (layer F.Cu) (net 16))
 (segment (start 144.37 111.42) (end 141.04101 108.09101) (width 0.25) (layer F.Cu) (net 16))
 (segment (start 141.04101 108.09101) (end 141.04101 106.59861) (width 0.25) (layer F.Cu) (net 16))
 (segment (start 139.8524 105.41) (end 139.7 105.41) (width 0.25) (layer F.Cu) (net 16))
 (segment (start 139.7 107.95) (end 139.8524 107.95) (width 0.25) (layer F.Cu) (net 17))
 (segment (start 139.8524 107.95) (end 143.9724 112.07) (width 0.25) (layer F.Cu) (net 17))
 (segment (start 143.9724 112.07) (end 144.37 112.07) (width 0.25) (layer F.Cu) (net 17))
 (segment (start 144.37 112.07) (end 144.995 112.07) (width 0.25) (layer F.Cu) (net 17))
 (segment (start 144.995 113.37) (end 142.7324 113.37) (width 0.25) (layer F.Cu) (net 18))
 (segment (start 142.7324 113.37) (end 139.8524 110.49) (width 0.25) (layer F.Cu) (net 18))
 (segment (start 139.8524 110.49) (end 139.7 110.49) (width 0.25) (layer F.Cu) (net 18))
 (segment (start 144.995 114.02) (end 140.69 114.02) (width 0.25) (layer F.Cu) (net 19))
 (segment (start 140.69 114.02) (end 139.7 113.03) (width 0.25) (layer F.Cu) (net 19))
 (segment (start 145.07 115.57) (end 145.07 116.72) (width 0.25) (layer B.Cu) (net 1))
 (segment (start 145.07 116.72) (end 144.315 117.475) (width 0.25) (layer B.Cu) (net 1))
 (via (at 144.315 117.475) (size 0.6) (drill 0.4) (layers F.Cu B.Cu) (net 1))
 (via (at 145.07 115.57) (size 0.6) (drill 0.4) (layers F.Cu B.Cu) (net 1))
 (segment (start 145.695 114.72) (end 145.695 114.945) (width 0.25) (layer F.Cu) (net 1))
 (segment (start 145.695 114.945) (end 145.07 115.57) (width 0.25) (layer F.Cu) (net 1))
 (segment (start 145.07 115.57) (end 140.966 115.57) (width 0.25) (layer F.Cu) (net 1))
 (segment (start 140.966 115.57) (end 139.7 115.57) (width 0.25) (layer F.Cu) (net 1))
 (segment (start 146.995 114.72) (end 146.995 115.345) (width 0.25) (layer F.Cu) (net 3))
 (segment (start 146.995 115.345) (end 146.040001 116.299999) (width 0.25) (layer F.Cu) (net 3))
 (segment (start 139.8524 118.11) (end 139.7 118.11) (width 0.25) (layer F.Cu) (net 3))
 (segment (start 146.040001 116.299999) (end 141.662401 116.299999) (width 0.25) (layer F.Cu) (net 3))
 (segment (start 141.662401 116.299999) (end 139.8524 118.11) (width 0.25) (layer F.Cu) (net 3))
 (segment (start 152.4 109.29) (end 152.4 105.2576) (width 0.25) (layer F.Cu) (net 10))
 (segment (start 152.4 105.2576) (end 154.7876 102.87) (width 0.25) (layer F.Cu) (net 10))
 (segment (start 154.7876 102.87) (end 154.94 102.87) (width 0.25) (layer F.Cu) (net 10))
 (segment (start 149.645 111.42) (end 150.27 111.42) (width 0.25) (layer F.Cu) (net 10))
 (segment (start 150.27 111.42) (end 152.4 109.29) (width 0.25) (layer F.Cu) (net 10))
 (segment (start 149.645 112.07) (end 150.27 112.07) (width 0.25) (layer F.Cu) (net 9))
 (segment (start 153.59899 108.74101) (end 153.59899 106.59861) (width 0.25) (layer F.Cu) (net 9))
 (segment (start 150.27 112.07) (end 153.59899 108.74101) (width 0.25) (layer F.Cu) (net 9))
 (segment (start 153.59899 106.59861) (end 154.7876 105.41) (width 0.25) (layer F.Cu) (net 9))
 (segment (start 154.7876 105.41) (end 154.94 105.41) (width 0.25) (layer F.Cu) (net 9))
 (segment (start 154.94 108.03641) (end 154.94 107.95) (width 0.25) (layer F.Cu) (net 8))
 (segment (start 153.674 109.966) (end 153.674 109.30241) (width 0.25) (layer F.Cu) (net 8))
 (segment (start 149.645 113.37) (end 150.27 113.37) (width 0.25) (layer F.Cu) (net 8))
 (segment (start 153.674 109.30241) (end 154.94 108.03641) (width 0.25) (layer F.Cu) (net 8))
 (segment (start 150.27 113.37) (end 153.674 109.966) (width 0.25) (layer F.Cu) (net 8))
 (segment (start 151.2576 114.02) (end 150.497415 113.259815) (width 0.25) (layer B.Cu) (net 7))
 (segment (start 149.72 107.696) (end 149.02 107.696) (width 0.25) (layer B.Cu) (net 7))
 (segment (start 150.497415 113.259815) (end 150.497415 108.473415) (width 0.25) (layer B.Cu) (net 7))
 (segment (start 150.497415 108.473415) (end 149.72 107.696) (width 0.25) (layer B.Cu) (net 7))
 (via (at 151.2576 114.02) (size 0.6) (drill 0.4) (layers F.Cu B.Cu) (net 7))
 (via (at 149.02 107.696) (size 0.6) (drill 0.4) (layers F.Cu B.Cu) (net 7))
 (segment (start 149.645 114.02) (end 151.2576 114.02) (width 0.25) (layer F.Cu) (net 7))
 (segment (start 151.2576 114.02) (end 154.7876 110.49) (width 0.25) (layer F.Cu) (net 7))
 (segment (start 154.7876 110.49) (end 154.94 110.49) (width 0.25) (layer F.Cu) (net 7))
 (segment (start 148.945 114.72) (end 153.0976 114.72) (width 0.25) (layer F.Cu) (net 6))
 (segment (start 153.0976 114.72) (end 154.7876 113.03) (width 0.25) (layer F.Cu) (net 6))
 (segment (start 154.7876 113.03) (end 154.94 113.03) (width 0.25) (layer F.Cu) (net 6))
 (segment (start 148.295 114.72) (end 148.295 115.345) (width 0.25) (layer F.Cu) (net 5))
 (segment (start 148.295 115.345) (end 148.52 115.57) (width 0.25) (layer F.Cu) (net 5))
 (segment (start 148.52 115.57) (end 153.674 115.57) (width 0.25) (layer F.Cu) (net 5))
 (segment (start 153.674 115.57) (end 154.94 115.57) (width 0.25) (layer F.Cu) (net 5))
 (segment (start 147.645 114.72) (end 147.645 115.345) (width 0.25) (layer F.Cu) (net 4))
 (segment (start 147.645 115.345) (end 148.599999 116.299999) (width 0.25) (layer F.Cu) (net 4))
 (segment (start 148.599999 116.299999) (end 152.977599 116.299999) (width 0.25) (layer F.Cu) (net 4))
 (segment (start 152.977599 116.299999) (end 154.7876 118.11) (width 0.25) (layer F.Cu) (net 4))
 (segment (start 154.7876 118.11) (end 154.94 118.11) (width 0.25) (layer F.Cu) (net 4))
 (segment (start 148.295 110.07) (end 148.295 109.445) (width 0.25) (layer F.Cu) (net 11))
 (segment (start 148.295 109.445) (end 148.868999 108.871001) (width 0.25) (layer F.Cu) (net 11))
 (segment (start 148.868999 108.871001) (end 149.730001 108.871001) (width 0.25) (layer F.Cu) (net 11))
 (segment (start 149.730001 108.871001) (end 151.13 107.471002) (width 0.25) (layer F.Cu) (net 11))
 (segment (start 151.13 107.471002) (end 151.13 105.89) (width 0.25) (layer F.Cu) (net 11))
 (segment (start 151.13 105.89) (end 151.13 105.14) (width 0.25) (layer F.Cu) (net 11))
 (segment (start 146.515 117.475) (end 148.275 117.475) (width 0.25) (layer F.Cu) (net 23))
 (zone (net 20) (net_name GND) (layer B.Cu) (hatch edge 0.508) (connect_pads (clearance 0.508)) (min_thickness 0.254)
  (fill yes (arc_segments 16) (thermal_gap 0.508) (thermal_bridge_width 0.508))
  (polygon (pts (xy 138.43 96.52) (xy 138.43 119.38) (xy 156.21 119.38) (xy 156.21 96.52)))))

